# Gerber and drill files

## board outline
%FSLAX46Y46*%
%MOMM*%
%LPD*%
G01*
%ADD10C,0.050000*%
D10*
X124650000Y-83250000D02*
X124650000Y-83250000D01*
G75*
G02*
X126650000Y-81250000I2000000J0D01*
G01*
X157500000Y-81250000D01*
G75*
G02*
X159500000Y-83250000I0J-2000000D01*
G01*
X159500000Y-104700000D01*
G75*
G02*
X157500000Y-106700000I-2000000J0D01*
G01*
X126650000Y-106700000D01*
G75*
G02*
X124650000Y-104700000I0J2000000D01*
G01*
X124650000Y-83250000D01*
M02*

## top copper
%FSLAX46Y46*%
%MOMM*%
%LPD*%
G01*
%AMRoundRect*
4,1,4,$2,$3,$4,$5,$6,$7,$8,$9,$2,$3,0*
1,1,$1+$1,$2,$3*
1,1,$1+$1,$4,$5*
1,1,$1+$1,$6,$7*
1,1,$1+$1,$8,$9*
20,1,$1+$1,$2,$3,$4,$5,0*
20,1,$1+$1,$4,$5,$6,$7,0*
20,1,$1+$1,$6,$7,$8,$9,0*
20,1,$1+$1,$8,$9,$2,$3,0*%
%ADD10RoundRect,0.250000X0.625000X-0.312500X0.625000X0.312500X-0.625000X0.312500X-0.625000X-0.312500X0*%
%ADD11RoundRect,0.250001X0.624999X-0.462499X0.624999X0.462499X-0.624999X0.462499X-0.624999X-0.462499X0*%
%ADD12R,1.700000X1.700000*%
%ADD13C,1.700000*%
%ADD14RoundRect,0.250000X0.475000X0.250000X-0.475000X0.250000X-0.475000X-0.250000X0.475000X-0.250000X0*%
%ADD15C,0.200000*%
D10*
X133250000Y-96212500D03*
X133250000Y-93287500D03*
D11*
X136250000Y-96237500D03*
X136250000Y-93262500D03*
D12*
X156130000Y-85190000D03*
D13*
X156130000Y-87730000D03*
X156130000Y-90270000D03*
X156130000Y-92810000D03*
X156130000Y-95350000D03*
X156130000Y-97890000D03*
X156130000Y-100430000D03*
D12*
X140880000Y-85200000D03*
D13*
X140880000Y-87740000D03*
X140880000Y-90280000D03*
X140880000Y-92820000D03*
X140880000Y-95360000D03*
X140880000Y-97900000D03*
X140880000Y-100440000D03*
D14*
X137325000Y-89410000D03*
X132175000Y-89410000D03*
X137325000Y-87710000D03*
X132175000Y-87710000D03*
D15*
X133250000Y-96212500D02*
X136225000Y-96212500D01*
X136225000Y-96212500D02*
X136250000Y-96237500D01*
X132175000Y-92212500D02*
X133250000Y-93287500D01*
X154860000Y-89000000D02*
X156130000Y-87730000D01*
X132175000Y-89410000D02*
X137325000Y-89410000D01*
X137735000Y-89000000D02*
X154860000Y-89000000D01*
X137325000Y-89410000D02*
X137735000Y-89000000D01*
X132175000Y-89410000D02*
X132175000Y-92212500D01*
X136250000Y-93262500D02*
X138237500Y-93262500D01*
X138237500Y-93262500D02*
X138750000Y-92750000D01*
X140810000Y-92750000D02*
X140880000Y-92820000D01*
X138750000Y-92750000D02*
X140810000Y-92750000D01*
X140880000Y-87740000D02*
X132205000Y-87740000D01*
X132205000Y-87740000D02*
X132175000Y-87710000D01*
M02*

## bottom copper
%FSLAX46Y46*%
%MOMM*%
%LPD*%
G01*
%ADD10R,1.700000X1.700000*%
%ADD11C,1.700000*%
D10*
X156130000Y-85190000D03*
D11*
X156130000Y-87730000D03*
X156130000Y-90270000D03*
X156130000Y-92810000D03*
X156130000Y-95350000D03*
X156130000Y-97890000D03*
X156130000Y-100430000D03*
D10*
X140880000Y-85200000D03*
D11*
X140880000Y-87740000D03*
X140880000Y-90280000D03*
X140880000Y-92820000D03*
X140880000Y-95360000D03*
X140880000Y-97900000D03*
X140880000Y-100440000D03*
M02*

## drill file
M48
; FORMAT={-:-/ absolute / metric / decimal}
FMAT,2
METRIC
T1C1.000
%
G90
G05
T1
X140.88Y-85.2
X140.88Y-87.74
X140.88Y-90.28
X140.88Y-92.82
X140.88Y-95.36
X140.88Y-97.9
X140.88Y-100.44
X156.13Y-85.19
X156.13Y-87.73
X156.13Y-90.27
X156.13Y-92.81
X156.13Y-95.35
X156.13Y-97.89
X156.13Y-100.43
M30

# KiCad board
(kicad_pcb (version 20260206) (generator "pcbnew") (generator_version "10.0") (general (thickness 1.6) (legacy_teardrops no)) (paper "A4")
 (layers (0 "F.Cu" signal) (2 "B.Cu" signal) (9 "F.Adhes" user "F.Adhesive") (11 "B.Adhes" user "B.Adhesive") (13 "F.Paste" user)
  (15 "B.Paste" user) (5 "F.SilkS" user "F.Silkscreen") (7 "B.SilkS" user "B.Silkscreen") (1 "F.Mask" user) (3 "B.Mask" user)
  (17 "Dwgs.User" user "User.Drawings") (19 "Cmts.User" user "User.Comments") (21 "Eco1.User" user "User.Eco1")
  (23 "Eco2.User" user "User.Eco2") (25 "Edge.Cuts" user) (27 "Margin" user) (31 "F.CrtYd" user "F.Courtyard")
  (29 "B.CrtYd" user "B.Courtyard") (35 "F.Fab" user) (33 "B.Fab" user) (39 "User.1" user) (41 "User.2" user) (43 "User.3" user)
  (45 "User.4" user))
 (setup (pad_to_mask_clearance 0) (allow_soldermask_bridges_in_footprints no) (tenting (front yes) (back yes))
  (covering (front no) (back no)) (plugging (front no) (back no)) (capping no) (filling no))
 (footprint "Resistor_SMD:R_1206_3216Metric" (layer "F.Cu") (at 133.25 94.75 90)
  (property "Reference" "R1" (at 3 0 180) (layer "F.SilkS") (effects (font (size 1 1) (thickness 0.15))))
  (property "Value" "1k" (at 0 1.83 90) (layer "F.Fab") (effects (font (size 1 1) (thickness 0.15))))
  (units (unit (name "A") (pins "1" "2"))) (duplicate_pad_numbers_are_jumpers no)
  (pad "1" smd roundrect (at -1.4625 0 90) (size 1.125 1.75) (layers "F.Cu" "F.Mask" "F.Paste") (roundrect_rratio 0.222222)
   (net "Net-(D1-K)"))
  (pad "2" smd roundrect (at 1.4625 0 90) (size 1.125 1.75) (layers "F.Cu" "F.Mask" "F.Paste") (roundrect_rratio 0.222222) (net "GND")))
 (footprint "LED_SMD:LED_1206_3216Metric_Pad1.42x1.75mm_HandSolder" (layer "F.Cu") (at 136.25 94.75 90)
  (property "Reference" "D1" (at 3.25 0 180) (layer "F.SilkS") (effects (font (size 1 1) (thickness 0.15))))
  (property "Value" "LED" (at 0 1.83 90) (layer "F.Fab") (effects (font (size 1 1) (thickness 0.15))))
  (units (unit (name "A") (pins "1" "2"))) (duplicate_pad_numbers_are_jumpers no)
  (pad "1" smd roundrect (at -1.4875 0 90) (size 1.425 1.75) (layers "F.Cu" "F.Mask" "F.Paste") (roundrect_rratio 0.175439)
   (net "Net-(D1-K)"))
  (pad "2" smd roundrect (at 1.4875 0 90) (size 1.425 1.75) (layers "F.Cu" "F.Mask" "F.Paste") (roundrect_rratio 0.175439)
   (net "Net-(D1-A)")))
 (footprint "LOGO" (layer "F.Cu") (at 132.075 102.575)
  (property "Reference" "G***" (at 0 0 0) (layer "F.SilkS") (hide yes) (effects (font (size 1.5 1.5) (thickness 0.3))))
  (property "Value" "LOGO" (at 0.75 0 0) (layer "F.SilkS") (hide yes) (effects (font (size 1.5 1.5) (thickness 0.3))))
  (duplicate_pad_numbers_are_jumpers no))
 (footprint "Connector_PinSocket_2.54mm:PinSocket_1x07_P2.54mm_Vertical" (layer "F.Cu") (at 156.13 85.19)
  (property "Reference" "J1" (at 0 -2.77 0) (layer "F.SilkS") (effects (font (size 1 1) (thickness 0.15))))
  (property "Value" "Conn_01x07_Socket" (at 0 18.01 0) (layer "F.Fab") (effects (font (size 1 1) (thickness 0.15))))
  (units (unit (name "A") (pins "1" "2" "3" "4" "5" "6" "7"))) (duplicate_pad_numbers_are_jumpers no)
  (pad "1" thru_hole rect (at 0 0) (size 1.7 1.7) (drill 1) (layers "*.Cu" "*.Mask") (remove_unused_layers no)
   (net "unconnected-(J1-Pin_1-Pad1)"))
  (pad "2" thru_hole circle (at 0 2.54) (size 1.7 1.7) (drill 1) (layers "*.Cu" "*.Mask") (remove_unused_layers no) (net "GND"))
  (pad "3" thru_hole circle (at 0 5.08) (size 1.7 1.7) (drill 1) (layers "*.Cu" "*.Mask") (remove_unused_layers no)
   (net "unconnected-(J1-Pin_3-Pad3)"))
  (pad "4" thru_hole circle (at 0 7.62) (size 1.7 1.7) (drill 1) (layers "*.Cu" "*.Mask") (remove_unused_layers no)
   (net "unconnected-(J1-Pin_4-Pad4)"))
  (pad "5" thru_hole circle (at 0 10.16) (size 1.7 1.7) (drill 1) (layers "*.Cu" "*.Mask") (remove_unused_layers no)
   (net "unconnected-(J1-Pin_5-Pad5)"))
  (pad "6" thru_hole circle (at 0 12.7) (size 1.7 1.7) (drill 1) (layers "*.Cu" "*.Mask") (remove_unused_layers no)
   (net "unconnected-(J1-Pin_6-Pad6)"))
  (pad "7" thru_hole circle (at 0 15.24) (size 1.7 1.7) (drill 1) (layers "*.Cu" "*.Mask") (remove_unused_layers no)
   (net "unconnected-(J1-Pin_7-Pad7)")))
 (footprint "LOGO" (layer "F.Cu") (at 128.375 93.5)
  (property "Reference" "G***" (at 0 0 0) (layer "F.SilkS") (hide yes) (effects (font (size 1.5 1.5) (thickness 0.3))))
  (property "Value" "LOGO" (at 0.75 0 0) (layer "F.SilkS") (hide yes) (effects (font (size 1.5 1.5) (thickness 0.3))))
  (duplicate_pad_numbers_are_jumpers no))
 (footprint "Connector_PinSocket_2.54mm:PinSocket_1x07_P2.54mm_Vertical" (layer "F.Cu") (at 140.88 85.2)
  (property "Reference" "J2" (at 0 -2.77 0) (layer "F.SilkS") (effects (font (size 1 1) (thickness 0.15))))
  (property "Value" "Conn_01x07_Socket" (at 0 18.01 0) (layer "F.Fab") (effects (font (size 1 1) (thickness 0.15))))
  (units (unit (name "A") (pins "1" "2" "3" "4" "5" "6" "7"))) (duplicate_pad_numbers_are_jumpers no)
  (pad "1" thru_hole rect (at 0 0) (size 1.7 1.7) (drill 1) (layers "*.Cu" "*.Mask") (remove_unused_layers no)
   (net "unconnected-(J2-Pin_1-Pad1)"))
  (pad "2" thru_hole circle (at 0 2.54) (size 1.7 1.7) (drill 1) (layers "*.Cu" "*.Mask") (remove_unused_layers no) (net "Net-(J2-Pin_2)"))
  (pad "3" thru_hole circle (at 0 5.08) (size 1.7 1.7) (drill 1) (layers "*.Cu" "*.Mask") (remove_unused_layers no)
   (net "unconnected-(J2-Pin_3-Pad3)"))
  (pad "4" thru_hole circle (at 0 7.62) (size 1.7 1.7) (drill 1) (layers "*.Cu" "*.Mask") (remove_unused_layers no) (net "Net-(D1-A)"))
  (pad "5" thru_hole circle (at 0 10.16) (size 1.7 1.7) (drill 1) (layers "*.Cu" "*.Mask") (remove_unused_layers no)
   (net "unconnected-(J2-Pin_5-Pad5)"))
  (pad "6" thru_hole circle (at 0 12.7) (size 1.7 1.7) (drill 1) (layers "*.Cu" "*.Mask") (remove_unused_layers no)
   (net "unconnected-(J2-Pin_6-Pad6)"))
  (pad "7" thru_hole circle (at 0 15.24) (size 1.7 1.7) (drill 1) (layers "*.Cu" "*.Mask") (remove_unused_layers no)
   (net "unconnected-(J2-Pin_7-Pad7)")))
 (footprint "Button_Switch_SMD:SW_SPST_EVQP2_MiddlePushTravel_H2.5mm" (layer "F.Cu") (at 134.75 88.56 180)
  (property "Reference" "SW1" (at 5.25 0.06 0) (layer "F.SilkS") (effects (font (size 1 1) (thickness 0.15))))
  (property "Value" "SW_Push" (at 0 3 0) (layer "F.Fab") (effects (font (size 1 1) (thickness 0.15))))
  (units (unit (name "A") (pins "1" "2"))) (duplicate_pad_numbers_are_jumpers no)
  (pad "1" smd roundrect (at -2.575 -0.85 180) (size 1.45 1) (layers "F.Cu" "F.Mask" "F.Paste") (roundrect_rratio 0.25) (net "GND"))
  (pad "1" smd roundrect (at 2.575 -0.85 180) (size 1.45 1) (layers "F.Cu" "F.Mask" "F.Paste") (roundrect_rratio 0.25) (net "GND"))
  (pad "2" smd roundrect (at -2.575 0.85 180) (size 1.45 1) (layers "F.Cu" "F.Mask" "F.Paste") (roundrect_rratio 0.25)
   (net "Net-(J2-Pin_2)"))
  (pad "2" smd roundrect (at 2.575 0.85 180) (size 1.45 1) (layers "F.Cu" "F.Mask" "F.Paste") (roundrect_rratio 0.25) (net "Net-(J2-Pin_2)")))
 (gr_rect (start 124.65 81.25) (end 159.5 106.7) (radius 2) (stroke (width 0.05) (type solid)) (fill no) (layer "Edge.Cuts"))
 (segment (start 133.25 96.2125) (end 136.225 96.2125) (width 0.2) (layer "F.Cu") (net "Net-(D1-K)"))
 (segment (start 136.225 96.2125) (end 136.25 96.2375) (width 0.2) (layer "F.Cu") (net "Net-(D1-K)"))
 (segment (start 132.175 92.2125) (end 133.25 93.2875) (width 0.2) (layer "F.Cu") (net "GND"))
 (segment (start 154.86 89) (end 156.13 87.73) (width 0.2) (layer "F.Cu") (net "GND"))
 (segment (start 132.175 89.41) (end 137.325 89.41) (width 0.2) (layer "F.Cu") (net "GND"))
 (segment (start 137.735 89) (end 154.86 89) (width 0.2) (layer "F.Cu") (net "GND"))
 (segment (start 137.325 89.41) (end 137.735 89) (width 0.2) (layer "F.Cu") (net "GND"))
 (segment (start 132.175 89.41) (end 132.175 92.2125) (width 0.2) (layer "F.Cu") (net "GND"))
 (segment (start 136.25 93.2625) (end 138.2375 93.2625) (width 0.2) (layer "F.Cu") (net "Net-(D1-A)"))
 (segment (start 138.2375 93.2625) (end 138.75 92.75) (width 0.2) (layer "F.Cu") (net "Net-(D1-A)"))
 (segment (start 140.81 92.75) (end 140.88 92.82) (width 0.2) (layer "F.Cu") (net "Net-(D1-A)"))
 (segment (start 138.75 92.75) (end 140.81 92.75) (width 0.2) (layer "F.Cu") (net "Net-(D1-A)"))
 (segment (start 140.88 87.74) (end 132.205 87.74) (width 0.2) (layer "F.Cu") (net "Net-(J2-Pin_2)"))
 (segment (start 132.205 87.74) (end 132.175 87.71) (width 0.2) (layer "F.Cu") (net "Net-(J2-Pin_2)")))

